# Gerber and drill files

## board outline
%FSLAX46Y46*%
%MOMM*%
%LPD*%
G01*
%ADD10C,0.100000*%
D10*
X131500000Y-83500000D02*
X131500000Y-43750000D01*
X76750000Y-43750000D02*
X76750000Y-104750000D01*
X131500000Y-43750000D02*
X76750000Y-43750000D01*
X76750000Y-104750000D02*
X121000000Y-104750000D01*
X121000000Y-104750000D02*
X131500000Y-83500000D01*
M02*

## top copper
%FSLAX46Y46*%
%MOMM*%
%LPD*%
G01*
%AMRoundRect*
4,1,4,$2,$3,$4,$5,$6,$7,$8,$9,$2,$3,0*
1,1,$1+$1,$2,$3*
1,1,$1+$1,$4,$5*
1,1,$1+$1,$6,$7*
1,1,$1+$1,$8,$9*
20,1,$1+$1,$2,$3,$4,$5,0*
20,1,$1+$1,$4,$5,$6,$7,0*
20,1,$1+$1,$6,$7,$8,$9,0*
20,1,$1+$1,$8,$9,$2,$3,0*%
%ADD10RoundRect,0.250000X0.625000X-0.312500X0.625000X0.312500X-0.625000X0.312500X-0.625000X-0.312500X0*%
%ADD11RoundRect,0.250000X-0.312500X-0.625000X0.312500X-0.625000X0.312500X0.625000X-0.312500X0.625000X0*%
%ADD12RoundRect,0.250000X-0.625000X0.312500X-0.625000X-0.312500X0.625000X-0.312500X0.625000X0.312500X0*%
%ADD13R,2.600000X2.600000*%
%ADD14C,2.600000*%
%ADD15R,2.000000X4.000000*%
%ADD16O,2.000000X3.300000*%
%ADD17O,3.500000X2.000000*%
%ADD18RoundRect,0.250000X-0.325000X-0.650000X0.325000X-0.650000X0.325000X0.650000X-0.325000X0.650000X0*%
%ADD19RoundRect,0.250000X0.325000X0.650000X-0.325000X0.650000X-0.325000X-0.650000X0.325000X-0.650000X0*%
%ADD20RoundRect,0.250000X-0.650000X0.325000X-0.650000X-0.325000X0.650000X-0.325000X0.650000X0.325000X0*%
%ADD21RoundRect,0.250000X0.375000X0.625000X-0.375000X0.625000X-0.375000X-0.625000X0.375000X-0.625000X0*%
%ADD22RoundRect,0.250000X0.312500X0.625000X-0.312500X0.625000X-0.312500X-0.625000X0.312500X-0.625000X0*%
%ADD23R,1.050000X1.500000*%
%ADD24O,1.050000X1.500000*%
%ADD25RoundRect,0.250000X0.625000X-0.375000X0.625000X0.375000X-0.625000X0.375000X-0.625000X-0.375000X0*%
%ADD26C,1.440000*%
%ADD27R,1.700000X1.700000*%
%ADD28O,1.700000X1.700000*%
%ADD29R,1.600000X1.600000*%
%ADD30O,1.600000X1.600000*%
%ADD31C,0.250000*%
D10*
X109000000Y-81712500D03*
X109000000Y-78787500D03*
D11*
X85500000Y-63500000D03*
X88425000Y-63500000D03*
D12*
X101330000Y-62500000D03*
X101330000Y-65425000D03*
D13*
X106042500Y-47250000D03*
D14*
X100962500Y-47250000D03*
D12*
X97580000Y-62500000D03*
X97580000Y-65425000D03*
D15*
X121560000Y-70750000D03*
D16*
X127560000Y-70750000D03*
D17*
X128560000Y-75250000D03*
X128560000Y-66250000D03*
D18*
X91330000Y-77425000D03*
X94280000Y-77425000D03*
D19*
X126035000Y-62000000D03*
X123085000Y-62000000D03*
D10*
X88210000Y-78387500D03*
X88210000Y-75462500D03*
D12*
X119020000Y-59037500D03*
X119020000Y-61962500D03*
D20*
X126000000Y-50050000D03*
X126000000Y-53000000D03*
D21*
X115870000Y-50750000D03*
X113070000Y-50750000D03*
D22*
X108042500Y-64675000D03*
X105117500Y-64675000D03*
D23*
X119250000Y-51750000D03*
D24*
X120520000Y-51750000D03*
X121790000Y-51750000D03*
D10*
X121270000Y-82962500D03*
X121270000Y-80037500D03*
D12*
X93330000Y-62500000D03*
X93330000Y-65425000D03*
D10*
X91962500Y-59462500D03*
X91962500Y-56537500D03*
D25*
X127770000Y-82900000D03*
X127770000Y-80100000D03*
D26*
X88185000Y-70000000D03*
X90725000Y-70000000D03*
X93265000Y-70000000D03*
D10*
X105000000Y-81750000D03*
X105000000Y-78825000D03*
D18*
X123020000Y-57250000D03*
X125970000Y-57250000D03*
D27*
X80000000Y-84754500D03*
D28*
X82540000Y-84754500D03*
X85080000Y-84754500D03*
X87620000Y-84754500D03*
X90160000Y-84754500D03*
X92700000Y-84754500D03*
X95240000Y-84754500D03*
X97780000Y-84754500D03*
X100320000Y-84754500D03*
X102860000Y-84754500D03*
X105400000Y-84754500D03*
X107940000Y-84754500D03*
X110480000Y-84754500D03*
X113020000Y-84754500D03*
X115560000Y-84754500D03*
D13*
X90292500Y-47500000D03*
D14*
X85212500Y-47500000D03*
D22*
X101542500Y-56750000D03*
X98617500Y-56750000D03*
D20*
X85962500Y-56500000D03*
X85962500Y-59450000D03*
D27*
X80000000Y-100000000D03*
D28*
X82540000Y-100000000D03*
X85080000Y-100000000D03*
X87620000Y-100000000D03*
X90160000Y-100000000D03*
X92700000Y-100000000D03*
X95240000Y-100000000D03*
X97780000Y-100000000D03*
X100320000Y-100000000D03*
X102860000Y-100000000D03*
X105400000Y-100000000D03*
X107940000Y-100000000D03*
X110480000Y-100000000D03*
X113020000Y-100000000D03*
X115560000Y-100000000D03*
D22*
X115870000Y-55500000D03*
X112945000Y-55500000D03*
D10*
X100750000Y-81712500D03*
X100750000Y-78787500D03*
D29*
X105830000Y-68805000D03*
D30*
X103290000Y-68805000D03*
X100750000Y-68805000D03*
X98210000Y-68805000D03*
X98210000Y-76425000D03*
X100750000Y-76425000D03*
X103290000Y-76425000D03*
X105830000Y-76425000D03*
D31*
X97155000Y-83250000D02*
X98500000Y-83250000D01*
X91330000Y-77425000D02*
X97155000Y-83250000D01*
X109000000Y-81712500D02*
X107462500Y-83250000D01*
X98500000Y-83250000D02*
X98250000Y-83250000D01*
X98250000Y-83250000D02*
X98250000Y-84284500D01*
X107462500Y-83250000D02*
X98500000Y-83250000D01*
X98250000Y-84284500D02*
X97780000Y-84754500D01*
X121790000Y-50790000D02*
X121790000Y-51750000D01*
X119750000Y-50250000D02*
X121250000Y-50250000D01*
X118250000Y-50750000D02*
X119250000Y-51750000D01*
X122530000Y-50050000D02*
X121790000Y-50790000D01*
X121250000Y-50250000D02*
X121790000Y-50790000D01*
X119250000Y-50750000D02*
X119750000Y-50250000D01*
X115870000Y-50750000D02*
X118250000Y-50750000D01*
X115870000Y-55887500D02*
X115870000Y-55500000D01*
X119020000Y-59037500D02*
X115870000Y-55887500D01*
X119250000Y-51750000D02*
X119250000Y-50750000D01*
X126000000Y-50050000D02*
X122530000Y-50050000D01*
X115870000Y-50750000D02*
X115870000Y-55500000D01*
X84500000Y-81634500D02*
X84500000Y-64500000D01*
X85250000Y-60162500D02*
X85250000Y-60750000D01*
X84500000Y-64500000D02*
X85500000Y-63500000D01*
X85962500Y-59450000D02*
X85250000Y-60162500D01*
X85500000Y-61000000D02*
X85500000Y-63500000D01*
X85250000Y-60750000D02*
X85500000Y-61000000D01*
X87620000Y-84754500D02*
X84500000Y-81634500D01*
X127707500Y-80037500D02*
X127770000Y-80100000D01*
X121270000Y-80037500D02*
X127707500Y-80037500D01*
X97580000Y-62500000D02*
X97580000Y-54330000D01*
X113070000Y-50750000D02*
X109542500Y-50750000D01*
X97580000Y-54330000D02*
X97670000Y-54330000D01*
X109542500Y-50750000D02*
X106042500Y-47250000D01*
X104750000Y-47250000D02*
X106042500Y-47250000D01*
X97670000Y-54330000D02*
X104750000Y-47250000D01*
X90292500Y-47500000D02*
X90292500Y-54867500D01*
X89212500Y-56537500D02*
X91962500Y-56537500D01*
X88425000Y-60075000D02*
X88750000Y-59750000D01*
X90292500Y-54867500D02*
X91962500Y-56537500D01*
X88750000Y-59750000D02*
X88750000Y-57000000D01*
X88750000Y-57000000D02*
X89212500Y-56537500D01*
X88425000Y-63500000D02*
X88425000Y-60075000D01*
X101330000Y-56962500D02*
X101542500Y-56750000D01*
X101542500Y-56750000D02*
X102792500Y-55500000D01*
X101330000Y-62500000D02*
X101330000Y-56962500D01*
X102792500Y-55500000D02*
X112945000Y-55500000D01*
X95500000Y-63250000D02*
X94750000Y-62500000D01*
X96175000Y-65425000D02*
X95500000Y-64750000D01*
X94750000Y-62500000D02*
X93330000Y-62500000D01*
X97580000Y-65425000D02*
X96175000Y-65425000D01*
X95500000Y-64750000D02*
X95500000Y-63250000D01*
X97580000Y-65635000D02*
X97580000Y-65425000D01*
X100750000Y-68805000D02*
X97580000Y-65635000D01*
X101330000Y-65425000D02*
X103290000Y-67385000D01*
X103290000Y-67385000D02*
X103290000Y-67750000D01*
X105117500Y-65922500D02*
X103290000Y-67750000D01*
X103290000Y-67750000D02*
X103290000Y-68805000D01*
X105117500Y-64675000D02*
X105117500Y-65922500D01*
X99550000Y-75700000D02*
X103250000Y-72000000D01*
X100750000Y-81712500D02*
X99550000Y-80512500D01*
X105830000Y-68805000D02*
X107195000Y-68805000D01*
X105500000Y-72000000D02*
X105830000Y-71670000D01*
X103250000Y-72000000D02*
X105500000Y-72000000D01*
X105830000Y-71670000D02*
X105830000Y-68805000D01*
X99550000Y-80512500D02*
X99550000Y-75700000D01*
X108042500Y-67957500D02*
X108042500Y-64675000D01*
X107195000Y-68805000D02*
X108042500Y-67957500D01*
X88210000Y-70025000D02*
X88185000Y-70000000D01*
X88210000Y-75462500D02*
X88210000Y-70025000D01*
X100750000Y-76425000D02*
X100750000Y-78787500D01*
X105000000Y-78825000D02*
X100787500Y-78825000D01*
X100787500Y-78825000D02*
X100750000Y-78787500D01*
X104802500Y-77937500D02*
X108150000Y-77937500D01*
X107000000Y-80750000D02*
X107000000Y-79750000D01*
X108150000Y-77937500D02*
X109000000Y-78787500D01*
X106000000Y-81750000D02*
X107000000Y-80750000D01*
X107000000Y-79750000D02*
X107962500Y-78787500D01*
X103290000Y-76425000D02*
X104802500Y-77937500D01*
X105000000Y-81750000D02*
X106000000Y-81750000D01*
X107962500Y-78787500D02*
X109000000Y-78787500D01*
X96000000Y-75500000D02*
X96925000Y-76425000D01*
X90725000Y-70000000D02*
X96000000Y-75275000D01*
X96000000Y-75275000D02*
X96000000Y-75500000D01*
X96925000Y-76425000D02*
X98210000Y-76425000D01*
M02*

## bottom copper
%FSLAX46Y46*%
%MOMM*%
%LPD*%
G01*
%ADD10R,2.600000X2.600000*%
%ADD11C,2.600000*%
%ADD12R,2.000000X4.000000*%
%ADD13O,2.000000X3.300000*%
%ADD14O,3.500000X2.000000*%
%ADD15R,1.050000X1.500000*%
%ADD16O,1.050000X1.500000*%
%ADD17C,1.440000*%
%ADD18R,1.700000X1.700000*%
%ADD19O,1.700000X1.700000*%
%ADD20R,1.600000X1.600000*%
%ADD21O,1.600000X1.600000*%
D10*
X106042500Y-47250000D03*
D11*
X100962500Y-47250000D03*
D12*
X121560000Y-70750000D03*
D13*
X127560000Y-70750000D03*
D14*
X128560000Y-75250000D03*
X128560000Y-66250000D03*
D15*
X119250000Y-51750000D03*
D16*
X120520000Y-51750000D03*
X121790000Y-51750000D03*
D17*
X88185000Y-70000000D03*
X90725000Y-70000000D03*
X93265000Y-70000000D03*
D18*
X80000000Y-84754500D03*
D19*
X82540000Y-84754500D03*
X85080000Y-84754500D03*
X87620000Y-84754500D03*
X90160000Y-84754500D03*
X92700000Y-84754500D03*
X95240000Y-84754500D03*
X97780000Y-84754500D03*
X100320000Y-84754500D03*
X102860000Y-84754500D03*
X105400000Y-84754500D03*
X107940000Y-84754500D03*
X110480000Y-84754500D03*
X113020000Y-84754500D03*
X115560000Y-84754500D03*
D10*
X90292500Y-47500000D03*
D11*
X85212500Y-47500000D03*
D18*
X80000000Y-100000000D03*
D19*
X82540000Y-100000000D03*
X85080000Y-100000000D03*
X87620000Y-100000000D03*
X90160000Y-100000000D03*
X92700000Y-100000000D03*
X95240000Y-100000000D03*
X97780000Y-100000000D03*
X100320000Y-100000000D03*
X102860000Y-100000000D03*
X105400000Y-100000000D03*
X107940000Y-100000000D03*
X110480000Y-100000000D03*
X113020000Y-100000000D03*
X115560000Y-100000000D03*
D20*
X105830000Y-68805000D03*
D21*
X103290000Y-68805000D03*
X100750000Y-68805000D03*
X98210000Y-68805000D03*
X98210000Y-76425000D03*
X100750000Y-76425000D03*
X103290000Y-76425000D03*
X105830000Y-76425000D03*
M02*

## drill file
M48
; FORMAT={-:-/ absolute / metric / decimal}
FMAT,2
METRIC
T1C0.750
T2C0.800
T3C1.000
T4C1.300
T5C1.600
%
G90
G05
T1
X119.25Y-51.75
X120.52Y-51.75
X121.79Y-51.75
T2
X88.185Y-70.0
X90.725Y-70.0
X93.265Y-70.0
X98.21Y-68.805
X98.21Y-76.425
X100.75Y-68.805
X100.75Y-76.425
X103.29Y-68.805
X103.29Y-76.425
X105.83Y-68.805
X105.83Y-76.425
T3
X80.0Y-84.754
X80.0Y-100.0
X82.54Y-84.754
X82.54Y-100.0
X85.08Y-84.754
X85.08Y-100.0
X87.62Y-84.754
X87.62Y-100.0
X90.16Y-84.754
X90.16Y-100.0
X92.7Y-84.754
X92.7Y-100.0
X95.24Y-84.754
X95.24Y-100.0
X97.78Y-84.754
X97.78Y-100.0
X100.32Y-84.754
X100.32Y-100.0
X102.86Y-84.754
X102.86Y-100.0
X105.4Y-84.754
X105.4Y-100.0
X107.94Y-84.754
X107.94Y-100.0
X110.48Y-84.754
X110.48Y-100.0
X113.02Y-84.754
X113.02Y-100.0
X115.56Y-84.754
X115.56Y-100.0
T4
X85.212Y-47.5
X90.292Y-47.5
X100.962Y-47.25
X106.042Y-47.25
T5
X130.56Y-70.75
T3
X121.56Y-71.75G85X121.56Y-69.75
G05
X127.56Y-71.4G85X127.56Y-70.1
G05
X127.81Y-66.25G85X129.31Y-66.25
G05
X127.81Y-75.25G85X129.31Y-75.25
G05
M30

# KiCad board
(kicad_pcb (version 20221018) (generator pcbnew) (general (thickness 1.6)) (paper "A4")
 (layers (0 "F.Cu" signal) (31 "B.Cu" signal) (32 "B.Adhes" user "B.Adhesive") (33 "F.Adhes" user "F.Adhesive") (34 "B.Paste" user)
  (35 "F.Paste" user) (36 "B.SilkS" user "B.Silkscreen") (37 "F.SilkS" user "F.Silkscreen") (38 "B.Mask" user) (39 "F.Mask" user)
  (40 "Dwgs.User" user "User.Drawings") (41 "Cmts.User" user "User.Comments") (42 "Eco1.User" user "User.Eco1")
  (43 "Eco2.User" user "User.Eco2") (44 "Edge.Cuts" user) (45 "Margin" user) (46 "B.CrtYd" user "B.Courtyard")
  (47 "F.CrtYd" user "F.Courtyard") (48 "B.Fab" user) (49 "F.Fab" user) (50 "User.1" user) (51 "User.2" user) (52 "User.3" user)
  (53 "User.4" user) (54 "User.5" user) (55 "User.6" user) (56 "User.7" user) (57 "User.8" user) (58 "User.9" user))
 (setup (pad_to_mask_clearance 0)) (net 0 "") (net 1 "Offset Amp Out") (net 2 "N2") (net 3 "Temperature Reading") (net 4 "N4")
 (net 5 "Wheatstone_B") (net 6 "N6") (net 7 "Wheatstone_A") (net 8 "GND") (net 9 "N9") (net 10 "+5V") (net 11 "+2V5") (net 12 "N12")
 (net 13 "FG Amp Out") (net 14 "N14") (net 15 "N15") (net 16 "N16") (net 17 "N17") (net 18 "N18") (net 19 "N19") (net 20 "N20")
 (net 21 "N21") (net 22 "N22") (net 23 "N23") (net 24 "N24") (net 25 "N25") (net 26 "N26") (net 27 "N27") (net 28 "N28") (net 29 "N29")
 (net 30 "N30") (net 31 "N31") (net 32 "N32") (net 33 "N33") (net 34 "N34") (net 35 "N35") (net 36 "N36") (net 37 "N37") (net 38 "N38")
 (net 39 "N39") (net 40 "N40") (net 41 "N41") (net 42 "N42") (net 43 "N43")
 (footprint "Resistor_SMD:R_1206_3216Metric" (layer "F.Cu") (at 109 80.25 90)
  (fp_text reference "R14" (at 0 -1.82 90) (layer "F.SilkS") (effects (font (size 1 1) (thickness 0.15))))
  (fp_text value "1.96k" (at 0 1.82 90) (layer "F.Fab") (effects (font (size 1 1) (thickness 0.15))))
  (pad "1" smd roundrect (at -1.4625 0 90) (size 1.125 1.75) (layers "F.Cu" "F.Paste" "F.Mask") (roundrect_rratio 0.222222)
   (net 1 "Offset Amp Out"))
  (pad "2" smd roundrect (at 1.4625 0 90) (size 1.125 1.75) (layers "F.Cu" "F.Paste" "F.Mask") (roundrect_rratio 0.222222) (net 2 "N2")))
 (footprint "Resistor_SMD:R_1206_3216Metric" (layer "F.Cu") (at 86.9625 63.5)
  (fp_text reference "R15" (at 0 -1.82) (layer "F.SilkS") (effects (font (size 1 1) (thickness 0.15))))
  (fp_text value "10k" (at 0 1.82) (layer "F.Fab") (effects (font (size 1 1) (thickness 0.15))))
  (pad "1" smd roundrect (at -1.4625 0) (size 1.125 1.75) (layers "F.Cu" "F.Paste" "F.Mask") (roundrect_rratio 0.222222)
   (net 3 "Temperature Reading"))
  (pad "2" smd roundrect (at 1.4625 0) (size 1.125 1.75) (layers "F.Cu" "F.Paste" "F.Mask") (roundrect_rratio 0.222222) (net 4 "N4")))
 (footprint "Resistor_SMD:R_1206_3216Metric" (layer "F.Cu") (at 101.33 63.9625 -90)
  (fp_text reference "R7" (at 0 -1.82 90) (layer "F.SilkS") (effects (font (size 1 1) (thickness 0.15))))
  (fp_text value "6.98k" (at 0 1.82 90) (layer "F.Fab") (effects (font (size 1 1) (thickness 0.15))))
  (pad "1" smd roundrect (at -1.4625 0 270) (size 1.125 1.75) (layers "F.Cu" "F.Paste" "F.Mask") (roundrect_rratio 0.222222)
   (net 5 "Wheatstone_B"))
  (pad "2" smd roundrect (at 1.4625 0 270) (size 1.125 1.75) (layers "F.Cu" "F.Paste" "F.Mask") (roundrect_rratio 0.222222) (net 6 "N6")))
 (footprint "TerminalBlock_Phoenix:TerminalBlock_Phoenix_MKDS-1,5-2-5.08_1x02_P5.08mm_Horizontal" (layer "F.Cu") (at 106.0425 47.25 180)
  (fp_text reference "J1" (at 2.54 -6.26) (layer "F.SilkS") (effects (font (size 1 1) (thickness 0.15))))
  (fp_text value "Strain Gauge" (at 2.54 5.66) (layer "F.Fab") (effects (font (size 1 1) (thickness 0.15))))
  (pad "1" thru_hole rect (at 0 0 180) (size 2.6 2.6) (drill 1.3) (layers "*.Cu" "*.Mask") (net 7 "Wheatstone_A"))
  (pad "2" thru_hole circle (at 5.08 0 180) (size 2.6 2.6) (drill 1.3) (layers "*.Cu" "*.Mask") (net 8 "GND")))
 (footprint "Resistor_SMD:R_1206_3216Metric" (layer "F.Cu") (at 97.58 63.9625 -90)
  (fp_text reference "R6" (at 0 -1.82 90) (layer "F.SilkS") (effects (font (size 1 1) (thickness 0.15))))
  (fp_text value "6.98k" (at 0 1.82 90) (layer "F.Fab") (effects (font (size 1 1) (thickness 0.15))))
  (pad "1" smd roundrect (at -1.4625 0 270) (size 1.125 1.75) (layers "F.Cu" "F.Paste" "F.Mask") (roundrect_rratio 0.222222)
   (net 7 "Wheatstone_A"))
  (pad "2" smd roundrect (at 1.4625 0 270) (size 1.125 1.75) (layers "F.Cu" "F.Paste" "F.Mask") (roundrect_rratio 0.222222) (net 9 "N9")))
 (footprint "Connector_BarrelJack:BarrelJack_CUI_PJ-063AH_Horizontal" (layer "F.Cu") (at 121.56 70.75 90)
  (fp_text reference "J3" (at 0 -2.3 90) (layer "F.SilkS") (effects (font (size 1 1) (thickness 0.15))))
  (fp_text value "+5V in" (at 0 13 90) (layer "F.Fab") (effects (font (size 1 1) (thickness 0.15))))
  (pad "" np_thru_hole circle (at 0 9 90) (size 1.6 1.6) (drill 1.6) (layers "*.Cu" "*.Mask"))
  (pad "1" thru_hole rect (at 0 0 90) (size 4 2) (drill oval 3 1) (layers "*.Cu" "*.Mask") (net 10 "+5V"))
  (pad "2" thru_hole oval (at 0 6 90) (size 3.3 2) (drill oval 2.3 1) (layers "*.Cu" "*.Mask") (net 8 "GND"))
  (pad "MP" thru_hole oval (at -4.5 7 90) (size 2 3.5) (drill oval 1 2.5) (layers "*.Cu" "*.Mask"))
  (pad "MP" thru_hole oval (at 4.5 7 90) (size 2 3.5) (drill oval 1 2.5) (layers "*.Cu" "*.Mask")))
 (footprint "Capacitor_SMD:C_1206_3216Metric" (layer "F.Cu") (at 92.805 77.425)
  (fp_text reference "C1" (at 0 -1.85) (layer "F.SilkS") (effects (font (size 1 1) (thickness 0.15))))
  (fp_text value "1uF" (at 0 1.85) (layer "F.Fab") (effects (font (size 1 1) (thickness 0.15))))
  (pad "1" smd roundrect (at -1.475 0) (size 1.15 1.8) (layers "F.Cu" "F.Paste" "F.Mask") (roundrect_rratio 0.217391)
   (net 1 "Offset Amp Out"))
  (pad "2" smd roundrect (at 1.475 0) (size 1.15 1.8) (layers "F.Cu" "F.Paste" "F.Mask") (roundrect_rratio 0.217391) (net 8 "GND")))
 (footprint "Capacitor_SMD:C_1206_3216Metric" (layer "F.Cu") (at 124.56 62 180)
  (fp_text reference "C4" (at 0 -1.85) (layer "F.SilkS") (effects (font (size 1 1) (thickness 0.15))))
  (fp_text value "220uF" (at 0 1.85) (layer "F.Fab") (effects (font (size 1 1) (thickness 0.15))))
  (pad "1" smd roundrect (at -1.475 0 180) (size 1.15 1.8) (layers "F.Cu" "F.Paste" "F.Mask") (roundrect_rratio 0.217391) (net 8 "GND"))
  (pad "2" smd roundrect (at 1.475 0 180) (size 1.15 1.8) (layers "F.Cu" "F.Paste" "F.Mask") (roundrect_rratio 0.217391) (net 10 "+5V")))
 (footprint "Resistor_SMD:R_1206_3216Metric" (layer "F.Cu") (at 88.21 76.925 90)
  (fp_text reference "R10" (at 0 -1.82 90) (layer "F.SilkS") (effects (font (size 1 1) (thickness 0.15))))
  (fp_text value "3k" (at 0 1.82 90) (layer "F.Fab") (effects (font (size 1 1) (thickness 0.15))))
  (pad "1" smd roundrect (at -1.4625 0 90) (size 1.125 1.75) (layers "F.Cu" "F.Paste" "F.Mask") (roundrect_rratio 0.222222) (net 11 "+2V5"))
  (pad "2" smd roundrect (at 1.4625 0 90) (size 1.125 1.75) (layers "F.Cu" "F.Paste" "F.Mask") (roundrect_rratio 0.222222) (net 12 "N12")))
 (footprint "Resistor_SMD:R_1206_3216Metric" (layer "F.Cu") (at 119.02 60.5 -90)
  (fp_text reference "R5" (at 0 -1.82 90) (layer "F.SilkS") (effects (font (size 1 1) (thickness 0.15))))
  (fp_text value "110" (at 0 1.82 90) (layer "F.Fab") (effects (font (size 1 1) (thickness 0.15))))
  (pad "1" smd roundrect (at -1.4625 0 270) (size 1.125 1.75) (layers "F.Cu" "F.Paste" "F.Mask") (roundrect_rratio 0.222222) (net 11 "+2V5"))
  (pad "2" smd roundrect (at 1.4625 0 270) (size 1.125 1.75) (layers "F.Cu" "F.Paste" "F.Mask") (roundrect_rratio 0.222222) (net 10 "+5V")))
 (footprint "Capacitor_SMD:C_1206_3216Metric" (layer "F.Cu") (at 126 51.525 -90)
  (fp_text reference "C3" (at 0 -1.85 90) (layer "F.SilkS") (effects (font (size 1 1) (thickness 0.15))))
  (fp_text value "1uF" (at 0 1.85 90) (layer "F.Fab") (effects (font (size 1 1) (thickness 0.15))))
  (pad "1" smd roundrect (at -1.475 0 270) (size 1.15 1.8) (layers "F.Cu" "F.Paste" "F.Mask") (roundrect_rratio 0.217391) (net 11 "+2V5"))
  (pad "2" smd roundrect (at 1.475 0 270) (size 1.15 1.8) (layers "F.Cu" "F.Paste" "F.Mask") (roundrect_rratio 0.217391) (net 8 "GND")))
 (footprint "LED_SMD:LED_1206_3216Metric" (layer "F.Cu") (at 114.47 50.75 180)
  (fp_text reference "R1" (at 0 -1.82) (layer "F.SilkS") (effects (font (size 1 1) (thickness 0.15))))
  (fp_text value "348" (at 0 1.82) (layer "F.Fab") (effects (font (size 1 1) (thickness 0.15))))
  (pad "1" smd roundrect (at -1.4 0 180) (size 1.25 1.75) (layers "F.Cu" "F.Paste" "F.Mask") (roundrect_rratio 0.2) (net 11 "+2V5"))
  (pad "2" smd roundrect (at 1.4 0 180) (size 1.25 1.75) (layers "F.Cu" "F.Paste" "F.Mask") (roundrect_rratio 0.2) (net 7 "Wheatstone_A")))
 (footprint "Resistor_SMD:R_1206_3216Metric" (layer "F.Cu") (at 106.58 64.675 180)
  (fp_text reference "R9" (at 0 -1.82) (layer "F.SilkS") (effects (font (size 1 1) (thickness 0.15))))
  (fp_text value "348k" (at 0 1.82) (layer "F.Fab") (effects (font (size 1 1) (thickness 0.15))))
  (pad "1" smd roundrect (at -1.4625 0 180) (size 1.125 1.75) (layers "F.Cu" "F.Paste" "F.Mask") (roundrect_rratio 0.222222)
   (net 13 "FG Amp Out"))
  (pad "2" smd roundrect (at 1.4625 0 180) (size 1.125 1.75) (layers "F.Cu" "F.Paste" "F.Mask") (roundrect_rratio 0.222222) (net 6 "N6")))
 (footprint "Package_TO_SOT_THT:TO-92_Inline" (layer "F.Cu") (at 119.25 51.75)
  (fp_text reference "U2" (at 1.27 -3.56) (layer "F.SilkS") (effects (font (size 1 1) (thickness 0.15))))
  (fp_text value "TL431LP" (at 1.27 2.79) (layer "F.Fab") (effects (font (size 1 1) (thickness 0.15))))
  (pad "1" thru_hole rect (at 0 0) (size 1.05 1.5) (drill 0.75) (layers "*.Cu" "*.Mask") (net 11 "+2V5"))
  (pad "2" thru_hole oval (at 1.27 0) (size 1.05 1.5) (drill 0.75) (layers "*.Cu" "*.Mask") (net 8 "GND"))
  (pad "3" thru_hole oval (at 2.54 0) (size 1.05 1.5) (drill 0.75) (layers "*.Cu" "*.Mask") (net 11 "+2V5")))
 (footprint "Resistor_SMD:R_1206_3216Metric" (layer "F.Cu") (at 121.27 81.5 90)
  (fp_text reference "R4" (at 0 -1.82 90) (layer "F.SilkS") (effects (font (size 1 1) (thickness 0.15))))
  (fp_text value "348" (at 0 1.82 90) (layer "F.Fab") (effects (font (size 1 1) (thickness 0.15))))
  (pad "1" smd roundrect (at -1.4625 0 90) (size 1.125 1.75) (layers "F.Cu" "F.Paste" "F.Mask") (roundrect_rratio 0.222222) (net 10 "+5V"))
  (pad "2" smd roundrect (at 1.4625 0 90) (size 1.125 1.75) (layers "F.Cu" "F.Paste" "F.Mask") (roundrect_rratio 0.222222) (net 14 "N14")))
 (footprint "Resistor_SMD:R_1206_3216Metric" (layer "F.Cu") (at 93.33 63.9625 -90)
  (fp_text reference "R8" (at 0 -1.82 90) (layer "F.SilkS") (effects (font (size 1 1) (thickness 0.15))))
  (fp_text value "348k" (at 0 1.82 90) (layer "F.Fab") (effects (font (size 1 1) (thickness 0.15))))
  (pad "1" smd roundrect (at -1.4625 0 270) (size 1.125 1.75) (layers "F.Cu" "F.Paste" "F.Mask") (roundrect_rratio 0.222222) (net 9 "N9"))
  (pad "2" smd roundrect (at 1.4625 0 270) (size 1.125 1.75) (layers "F.Cu" "F.Paste" "F.Mask") (roundrect_rratio 0.222222) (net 8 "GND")))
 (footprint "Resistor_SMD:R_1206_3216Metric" (layer "F.Cu") (at 91.9625 58 90)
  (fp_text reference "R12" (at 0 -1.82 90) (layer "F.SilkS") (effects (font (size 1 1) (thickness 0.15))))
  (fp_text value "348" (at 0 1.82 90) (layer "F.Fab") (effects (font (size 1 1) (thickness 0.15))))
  (pad "1" smd roundrect (at -1.4625 0 90) (size 1.125 1.75) (layers "F.Cu" "F.Paste" "F.Mask") (roundrect_rratio 0.222222) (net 10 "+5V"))
  (pad "2" smd roundrect (at 1.4625 0 90) (size 1.125 1.75) (layers "F.Cu" "F.Paste" "F.Mask") (roundrect_rratio 0.222222) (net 4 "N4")))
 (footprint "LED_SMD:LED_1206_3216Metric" (layer "F.Cu") (at 127.77 81.5 90)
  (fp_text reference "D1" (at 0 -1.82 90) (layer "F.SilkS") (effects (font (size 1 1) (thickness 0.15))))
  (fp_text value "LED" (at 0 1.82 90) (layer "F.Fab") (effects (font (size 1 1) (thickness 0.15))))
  (pad "1" smd roundrect (at -1.4 0 90) (size 1.25 1.75) (layers "F.Cu" "F.Paste" "F.Mask") (roundrect_rratio 0.2) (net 8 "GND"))
  (pad "2" smd roundrect (at 1.4 0 90) (size 1.25 1.75) (layers "F.Cu" "F.Paste" "F.Mask") (roundrect_rratio 0.2) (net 14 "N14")))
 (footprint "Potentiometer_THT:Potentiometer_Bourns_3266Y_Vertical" (layer "F.Cu") (at 88.185 70 180)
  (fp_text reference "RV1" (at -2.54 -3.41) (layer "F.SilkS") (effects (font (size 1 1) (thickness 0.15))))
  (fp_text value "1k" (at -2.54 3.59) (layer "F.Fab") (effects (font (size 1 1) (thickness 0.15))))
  (pad "1" thru_hole circle (at 0 0 180) (size 1.44 1.44) (drill 0.8) (layers "*.Cu" "*.Mask") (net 12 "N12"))
  (pad "2" thru_hole circle (at -2.54 0 180) (size 1.44 1.44) (drill 0.8) (layers "*.Cu" "*.Mask") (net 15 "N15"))
  (pad "3" thru_hole circle (at -5.08 0 180) (size 1.44 1.44) (drill 0.8) (layers "*.Cu" "*.Mask") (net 8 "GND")))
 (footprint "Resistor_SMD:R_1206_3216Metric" (layer "F.Cu") (at 105 80.2875 90)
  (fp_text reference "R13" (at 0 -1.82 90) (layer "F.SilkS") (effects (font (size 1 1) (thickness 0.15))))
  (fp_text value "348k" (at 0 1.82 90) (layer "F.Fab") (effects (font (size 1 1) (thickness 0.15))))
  (pad "1" smd roundrect (at -1.4625 0 90) (size 1.125 1.75) (layers "F.Cu" "F.Paste" "F.Mask") (roundrect_rratio 0.222222) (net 2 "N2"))
  (pad "2" smd roundrect (at 1.4625 0 90) (size 1.125 1.75) (layers "F.Cu" "F.Paste" "F.Mask") (roundrect_rratio 0.222222) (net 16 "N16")))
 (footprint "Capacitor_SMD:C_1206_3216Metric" (layer "F.Cu") (at 124.495 57.25)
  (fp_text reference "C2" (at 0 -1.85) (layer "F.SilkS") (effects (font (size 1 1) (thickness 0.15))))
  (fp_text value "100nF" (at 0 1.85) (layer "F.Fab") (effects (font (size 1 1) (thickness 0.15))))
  (pad "1" smd roundrect (at -1.475 0) (size 1.15 1.8) (layers "F.Cu" "F.Paste" "F.Mask") (roundrect_rratio 0.217391) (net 10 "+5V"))
  (pad "2" smd roundrect (at 1.475 0) (size 1.15 1.8) (layers "F.Cu" "F.Paste" "F.Mask") (roundrect_rratio 0.217391) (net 8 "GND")))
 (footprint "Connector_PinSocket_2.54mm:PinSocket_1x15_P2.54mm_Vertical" (layer "F.Cu") (at 80 84.7545 90)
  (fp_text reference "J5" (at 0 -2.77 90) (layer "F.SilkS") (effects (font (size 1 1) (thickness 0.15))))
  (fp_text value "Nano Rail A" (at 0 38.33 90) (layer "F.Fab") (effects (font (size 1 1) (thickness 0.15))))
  (pad "1" thru_hole rect (at 0 0 90) (size 1.7 1.7) (drill 1) (layers "*.Cu" "*.Mask") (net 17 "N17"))
  (pad "2" thru_hole oval (at 0 2.54 90) (size 1.7 1.7) (drill 1) (layers "*.Cu" "*.Mask") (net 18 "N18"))
  (pad "3" thru_hole oval (at 0 5.08 90) (size 1.7 1.7) (drill 1) (layers "*.Cu" "*.Mask") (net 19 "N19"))
  (pad "4" thru_hole oval (at 0 7.62 90) (size 1.7 1.7) (drill 1) (layers "*.Cu" "*.Mask") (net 3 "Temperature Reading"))
  (pad "5" thru_hole oval (at 0 10.16 90) (size 1.7 1.7) (drill 1) (layers "*.Cu" "*.Mask") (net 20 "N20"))
  (pad "6" thru_hole oval (at 0 12.7 90) (size 1.7 1.7) (drill 1) (layers "*.Cu" "*.Mask") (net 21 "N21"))
  (pad "7" thru_hole oval (at 0 15.24 90) (size 1.7 1.7) (drill 1) (layers "*.Cu" "*.Mask") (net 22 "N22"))
  (pad "8" thru_hole oval (at 0 17.78 90) (size 1.7 1.7) (drill 1) (layers "*.Cu" "*.Mask") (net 1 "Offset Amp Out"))
  (pad "9" thru_hole oval (at 0 20.32 90) (size 1.7 1.7) (drill 1) (layers "*.Cu" "*.Mask") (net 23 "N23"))
  (pad "10" thru_hole oval (at 0 22.86 90) (size 1.7 1.7) (drill 1) (layers "*.Cu" "*.Mask") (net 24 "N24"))
  (pad "11" thru_hole oval (at 0 25.4 90) (size 1.7 1.7) (drill 1) (layers "*.Cu" "*.Mask") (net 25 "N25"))
  (pad "12" thru_hole oval (at 0 27.94 90) (size 1.7 1.7) (drill 1) (layers "*.Cu" "*.Mask") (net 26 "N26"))
  (pad "13" thru_hole oval (at 0 30.48 90) (size 1.7 1.7) (drill 1) (layers "*.Cu" "*.Mask") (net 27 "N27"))
  (pad "14" thru_hole oval (at 0 33.02 90) (size 1.7 1.7) (drill 1) (layers "*.Cu" "*.Mask") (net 8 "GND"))
  (pad "15" thru_hole oval (at 0 35.56 90) (size 1.7 1.7) (drill 1) (layers "*.Cu" "*.Mask") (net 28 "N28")))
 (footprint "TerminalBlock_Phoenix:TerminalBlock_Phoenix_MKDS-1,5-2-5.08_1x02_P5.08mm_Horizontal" (layer "F.Cu") (at 90.2925 47.5 180)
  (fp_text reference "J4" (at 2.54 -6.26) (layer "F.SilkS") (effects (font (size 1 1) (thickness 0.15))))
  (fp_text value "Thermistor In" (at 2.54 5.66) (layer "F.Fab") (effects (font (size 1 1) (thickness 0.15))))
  (pad "1" thru_hole rect (at 0 0 180) (size 2.6 2.6) (drill 1.3) (layers "*.Cu" "*.Mask") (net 4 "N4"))
  (pad "2" thru_hole circle (at 5.08 0 180) (size 2.6 2.6) (drill 1.3) (layers "*.Cu" "*.Mask") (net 8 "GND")))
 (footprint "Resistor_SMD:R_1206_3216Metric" (layer "F.Cu") (at 100.08 56.75 180)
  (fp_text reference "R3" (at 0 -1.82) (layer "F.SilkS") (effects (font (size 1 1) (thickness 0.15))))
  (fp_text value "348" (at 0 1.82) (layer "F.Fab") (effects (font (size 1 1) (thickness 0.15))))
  (pad "1" smd roundrect (at -1.4625 0 180) (size 1.125 1.75) (layers "F.Cu" "F.Paste" "F.Mask") (roundrect_rratio 0.222222)
   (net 5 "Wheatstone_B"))
  (pad "2" smd roundrect (at 1.4625 0 180) (size 1.125 1.75) (layers "F.Cu" "F.Paste" "F.Mask") (roundrect_rratio 0.222222) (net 8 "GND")))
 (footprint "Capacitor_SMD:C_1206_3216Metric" (layer "F.Cu") (at 85.9625 57.975 -90)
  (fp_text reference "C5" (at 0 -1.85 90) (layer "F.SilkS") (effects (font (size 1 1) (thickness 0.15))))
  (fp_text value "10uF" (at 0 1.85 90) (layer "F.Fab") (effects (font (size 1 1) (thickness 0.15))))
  (pad "1" smd roundrect (at -1.475 0 270) (size 1.15 1.8) (layers "F.Cu" "F.Paste" "F.Mask") (roundrect_rratio 0.217391) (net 8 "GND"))
  (pad "2" smd roundrect (at 1.475 0 270) (size 1.15 1.8) (layers "F.Cu" "F.Paste" "F.Mask") (roundrect_rratio 0.217391)
   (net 3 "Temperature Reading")))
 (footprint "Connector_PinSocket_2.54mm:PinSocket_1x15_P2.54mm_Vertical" (layer "F.Cu") (at 80 100 90)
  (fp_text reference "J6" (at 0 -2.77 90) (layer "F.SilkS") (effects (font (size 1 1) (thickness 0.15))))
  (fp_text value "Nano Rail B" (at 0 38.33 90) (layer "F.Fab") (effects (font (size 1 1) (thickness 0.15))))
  (pad "1" thru_hole rect (at 0 0 90) (size 1.7 1.7) (drill 1) (layers "*.Cu" "*.Mask") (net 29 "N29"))
  (pad "2" thru_hole oval (at 0 2.54 90) (size 1.7 1.7) (drill 1) (layers "*.Cu" "*.Mask") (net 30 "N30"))
  (pad "3" thru_hole oval (at 0 5.08 90) (size 1.7 1.7) (drill 1) (layers "*.Cu" "*.Mask") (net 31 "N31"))
  (pad "4" thru_hole oval (at 0 7.62 90) (size 1.7 1.7) (drill 1) (layers "*.Cu" "*.Mask") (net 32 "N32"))
  (pad "5" thru_hole oval (at 0 10.16 90) (size 1.7 1.7) (drill 1) (layers "*.Cu" "*.Mask") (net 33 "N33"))
  (pad "6" thru_hole oval (at 0 12.7 90) (size 1.7 1.7) (drill 1) (layers "*.Cu" "*.Mask") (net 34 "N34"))
  (pad "7" thru_hole oval (at 0 15.24 90) (size 1.7 1.7) (drill 1) (layers "*.Cu" "*.Mask") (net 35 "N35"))
  (pad "8" thru_hole oval (at 0 17.78 90) (size 1.7 1.7) (drill 1) (layers "*.Cu" "*.Mask") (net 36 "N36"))
  (pad "9" thru_hole oval (at 0 20.32 90) (size 1.7 1.7) (drill 1) (layers "*.Cu" "*.Mask") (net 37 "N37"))
  (pad "10" thru_hole oval (at 0 22.86 90) (size 1.7 1.7) (drill 1) (layers "*.Cu" "*.Mask") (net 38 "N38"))
  (pad "11" thru_hole oval (at 0 25.4 90) (size 1.7 1.7) (drill 1) (layers "*.Cu" "*.Mask") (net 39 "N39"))
  (pad "12" thru_hole oval (at 0 27.94 90) (size 1.7 1.7) (drill 1) (layers "*.Cu" "*.Mask") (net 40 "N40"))
  (pad "13" thru_hole oval (at 0 30.48 90) (size 1.7 1.7) (drill 1) (layers "*.Cu" "*.Mask") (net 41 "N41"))
  (pad "14" thru_hole oval (at 0 33.02 90) (size 1.7 1.7) (drill 1) (layers "*.Cu" "*.Mask") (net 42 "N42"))
  (pad "15" thru_hole oval (at 0 35.56 90) (size 1.7 1.7) (drill 1) (layers "*.Cu" "*.Mask") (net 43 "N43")))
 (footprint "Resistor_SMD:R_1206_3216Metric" (layer "F.Cu") (at 114.4075 55.5 180)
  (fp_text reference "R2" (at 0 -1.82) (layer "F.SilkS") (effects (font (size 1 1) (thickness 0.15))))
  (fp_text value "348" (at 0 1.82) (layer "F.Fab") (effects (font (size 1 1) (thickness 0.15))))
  (pad "1" smd roundrect (at -1.4625 0 180) (size 1.125 1.75) (layers "F.Cu" "F.Paste" "F.Mask") (roundrect_rratio 0.222222) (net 11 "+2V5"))
  (pad "2" smd roundrect (at 1.4625 0 180) (size 1.125 1.75) (layers "F.Cu" "F.Paste" "F.Mask") (roundrect_rratio 0.222222)
   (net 5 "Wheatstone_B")))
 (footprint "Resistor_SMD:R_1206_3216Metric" (layer "F.Cu") (at 100.75 80.25 90)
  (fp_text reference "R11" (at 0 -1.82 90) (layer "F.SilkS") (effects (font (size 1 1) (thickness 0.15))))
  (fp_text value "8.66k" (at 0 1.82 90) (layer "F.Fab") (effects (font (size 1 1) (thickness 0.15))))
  (pad "1" smd roundrect (at -1.4625 0 90) (size 1.125 1.75) (layers "F.Cu" "F.Paste" "F.Mask") (roundrect_rratio 0.222222)
   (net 13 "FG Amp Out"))
  (pad "2" smd roundrect (at 1.4625 0 90) (size 1.125 1.75) (layers "F.Cu" "F.Paste" "F.Mask") (roundrect_rratio 0.222222) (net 16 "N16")))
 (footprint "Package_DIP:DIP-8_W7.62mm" (layer "F.Cu") (at 105.83 68.805 -90)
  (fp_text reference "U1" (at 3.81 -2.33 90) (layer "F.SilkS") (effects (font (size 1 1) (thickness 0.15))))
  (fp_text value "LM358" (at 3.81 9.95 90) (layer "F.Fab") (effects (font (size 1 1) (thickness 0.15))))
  (pad "1" thru_hole rect (at 0 0 270) (size 1.6 1.6) (drill 0.8) (layers "*.Cu" "*.Mask") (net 13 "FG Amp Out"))
  (pad "2" thru_hole oval (at 0 2.54 270) (size 1.6 1.6) (drill 0.8) (layers "*.Cu" "*.Mask") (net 6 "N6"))
  (pad "3" thru_hole oval (at 0 5.08 270) (size 1.6 1.6) (drill 0.8) (layers "*.Cu" "*.Mask") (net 9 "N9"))
  (pad "4" thru_hole oval (at 0 7.62 270) (size 1.6 1.6) (drill 0.8) (layers "*.Cu" "*.Mask") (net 8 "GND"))
  (pad "5" thru_hole oval (at 7.62 7.62 270) (size 1.6 1.6) (drill 0.8) (layers "*.Cu" "*.Mask") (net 15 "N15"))
  (pad "6" thru_hole oval (at 7.62 5.08 270) (size 1.6 1.6) (drill 0.8) (layers "*.Cu" "*.Mask") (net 16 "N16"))
  (pad "7" thru_hole oval (at 7.62 2.54 270) (size 1.6 1.6) (drill 0.8) (layers "*.Cu" "*.Mask") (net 2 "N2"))
  (pad "8" thru_hole oval (at 7.62 0 270) (size 1.6 1.6) (drill 0.8) (layers "*.Cu" "*.Mask") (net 10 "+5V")))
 (gr_line (start 131.5 83.5) (end 131.5 43.75) (stroke (width 0.1) (type default)) (layer "Edge.Cuts"))
 (gr_line (start 76.75 43.75) (end 76.75 104.75) (stroke (width 0.1) (type default)) (layer "Edge.Cuts"))
 (gr_line (start 131.5 43.75) (end 76.75 43.75) (stroke (width 0.1) (type default)) (layer "Edge.Cuts"))
 (gr_line (start 76.75 104.75) (end 121 104.75) (stroke (width 0.1) (type default)) (layer "Edge.Cuts"))
 (gr_line (start 121 104.75) (end 131.5 83.5) (stroke (width 0.1) (type default)) (layer "Edge.Cuts"))
 (segment (start 97.155 83.25) (end 98.5 83.25) (width 0.25) (layer "F.Cu") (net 1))
 (segment (start 91.33 77.425) (end 97.155 83.25) (width 0.25) (layer "F.Cu") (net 1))
 (segment (start 109 81.7125) (end 107.4625 83.25) (width 0.25) (layer "F.Cu") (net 1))
 (segment (start 98.5 83.25) (end 98.25 83.25) (width 0.25) (layer "F.Cu") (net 1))
 (segment (start 98.25 83.25) (end 98.25 84.2845) (width 0.25) (layer "F.Cu") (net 1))
 (segment (start 107.4625 83.25) (end 98.5 83.25) (width 0.25) (layer "F.Cu") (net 1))
 (segment (start 98.25 84.2845) (end 97.78 84.7545) (width 0.25) (layer "F.Cu") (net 1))
 (segment (start 121.79 50.79) (end 121.79 51.75) (width 0.25) (layer "F.Cu") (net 11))
 (segment (start 119.75 50.25) (end 121.25 50.25) (width 0.25) (layer "F.Cu") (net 11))
 (segment (start 118.25 50.75) (end 119.25 51.75) (width 0.25) (layer "F.Cu") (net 11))
 (segment (start 122.53 50.05) (end 121.79 50.79) (width 0.25) (layer "F.Cu") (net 11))
 (segment (start 121.25 50.25) (end 121.79 50.79) (width 0.25) (layer "F.Cu") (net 11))
 (segment (start 119.25 50.75) (end 119.75 50.25) (width 0.25) (layer "F.Cu") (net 11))
 (segment (start 115.87 50.75) (end 118.25 50.75) (width 0.25) (layer "F.Cu") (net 11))
 (segment (start 115.87 55.8875) (end 115.87 55.5) (width 0.25) (layer "F.Cu") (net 11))
 (segment (start 119.02 59.0375) (end 115.87 55.8875) (width 0.25) (layer "F.Cu") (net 11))
 (segment (start 119.25 51.75) (end 119.25 50.75) (width 0.25) (layer "F.Cu") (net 11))
 (segment (start 126 50.05) (end 122.53 50.05) (width 0.25) (layer "F.Cu") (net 11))
 (segment (start 115.87 50.75) (end 115.87 55.5) (width 0.25) (layer "F.Cu") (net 11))
 (segment (start 84.5 81.6345) (end 84.5 64.5) (width 0.25) (layer "F.Cu") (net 3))
 (segment (start 85.25 60.1625) (end 85.25 60.75) (width 0.25) (layer "F.Cu") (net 3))
 (segment (start 84.5 64.5) (end 85.5 63.5) (width 0.25) (layer "F.Cu") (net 3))
 (segment (start 85.9625 59.45) (end 85.25 60.1625) (width 0.25) (layer "F.Cu") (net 3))
 (segment (start 85.5 61) (end 85.5 63.5) (width 0.25) (layer "F.Cu") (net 3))
 (segment (start 85.25 60.75) (end 85.5 61) (width 0.25) (layer "F.Cu") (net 3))
 (segment (start 87.62 84.7545) (end 84.5 81.6345) (width 0.25) (layer "F.Cu") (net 3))
 (segment (start 127.7075 80.0375) (end 127.77 80.1) (width 0.25) (layer "F.Cu") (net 14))
 (segment (start 121.27 80.0375) (end 127.7075 80.0375) (width 0.25) (layer "F.Cu") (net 14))
 (segment (start 97.58 62.5) (end 97.58 54.33) (width 0.25) (layer "F.Cu") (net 7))
 (segment (start 113.07 50.75) (end 109.5425 50.75) (width 0.25) (layer "F.Cu") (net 7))
 (segment (start 97.58 54.33) (end 97.67 54.33) (width 0.25) (layer "F.Cu") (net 7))
 (segment (start 109.5425 50.75) (end 106.0425 47.25) (width 0.25) (layer "F.Cu") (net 7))
 (segment (start 104.75 47.25) (end 106.0425 47.25) (width 0.25) (layer "F.Cu") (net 7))
 (segment (start 97.67 54.33) (end 104.75 47.25) (width 0.25) (layer "F.Cu") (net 7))
 (segment (start 90.2925 47.5) (end 90.2925 54.8675) (width 0.25) (layer "F.Cu") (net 4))
 (segment (start 89.2125 56.5375) (end 91.9625 56.5375) (width 0.25) (layer "F.Cu") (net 4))
 (segment (start 88.425 60.075) (end 88.75 59.75) (width 0.25) (layer "F.Cu") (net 4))
 (segment (start 90.2925 54.8675) (end 91.9625 56.5375) (width 0.25) (layer "F.Cu") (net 4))
 (segment (start 88.75 59.75) (end 88.75 57) (width 0.25) (layer "F.Cu") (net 4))
 (segment (start 88.75 57) (end 89.2125 56.5375) (width 0.25) (layer "F.Cu") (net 4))
 (segment (start 88.425 63.5) (end 88.425 60.075) (width 0.25) (layer "F.Cu") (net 4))
 (segment (start 101.33 56.9625) (end 101.5425 56.75) (width 0.25) (layer "F.Cu") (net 5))
 (segment (start 101.5425 56.75) (end 102.7925 55.5) (width 0.25) (layer "F.Cu") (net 5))
 (segment (start 101.33 62.5) (end 101.33 56.9625) (width 0.25) (layer "F.Cu") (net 5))
 (segment (start 102.7925 55.5) (end 112.945 55.5) (width 0.25) (layer "F.Cu") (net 5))
 (segment (start 95.5 63.25) (end 94.75 62.5) (width 0.25) (layer "F.Cu") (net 9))
 (segment (start 96.175 65.425) (end 95.5 64.75) (width 0.25) (layer "F.Cu") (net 9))
 (segment (start 94.75 62.5) (end 93.33 62.5) (width 0.25) (layer "F.Cu") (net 9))
 (segment (start 97.58 65.425) (end 96.175 65.425) (width 0.25) (layer "F.Cu") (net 9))
 (segment (start 95.5 64.75) (end 95.5 63.25) (width 0.25) (layer "F.Cu") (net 9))
 (segment (start 97.58 65.635) (end 97.58 65.425) (width 0.25) (layer "F.Cu") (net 9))
 (segment (start 100.75 68.805) (end 97.58 65.635) (width 0.25) (layer "F.Cu") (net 9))
 (segment (start 101.33 65.425) (end 103.29 67.385) (width 0.25) (layer "F.Cu") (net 6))
 (segment (start 103.29 67.385) (end 103.29 67.75) (width 0.25) (layer "F.Cu") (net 6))
 (segment (start 105.1175 65.9225) (end 103.29 67.75) (width 0.25) (layer "F.Cu") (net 6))
 (segment (start 103.29 67.75) (end 103.29 68.805) (width 0.25) (layer "F.Cu") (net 6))
 (segment (start 105.1175 64.675) (end 105.1175 65.9225) (width 0.25) (layer "F.Cu") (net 6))
 (segment (start 99.55 75.7) (end 103.25 72) (width 0.25) (layer "F.Cu") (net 13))
 (segment (start 100.75 81.7125) (end 99.55 80.5125) (width 0.25) (layer "F.Cu") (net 13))
 (segment (start 105.83 68.805) (end 107.195 68.805) (width 0.25) (layer "F.Cu") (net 13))
 (segment (start 105.5 72) (end 105.83 71.67) (width 0.25) (layer "F.Cu") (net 13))
 (segment (start 103.25 72) (end 105.5 72) (width 0.25) (layer "F.Cu") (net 13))
 (segment (start 105.83 71.67) (end 105.83 68.805) (width 0.25) (layer "F.Cu") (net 13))
 (segment (start 99.55 80.5125) (end 99.55 75.7) (width 0.25) (layer "F.Cu") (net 13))
 (segment (start 108.0425 67.9575) (end 108.0425 64.675) (width 0.25) (layer "F.Cu") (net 13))
 (segment (start 107.195 68.805) (end 108.0425 67.9575) (width 0.25) (layer "F.Cu") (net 13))
 (segment (start 88.21 70.025) (end 88.185 70) (width 0.25) (layer "F.Cu") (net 12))
 (segment (start 88.21 75.4625) (end 88.21 70.025) (width 0.25) (layer "F.Cu") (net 12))
 (segment (start 100.75 76.425) (end 100.75 78.7875) (width 0.25) (layer "F.Cu") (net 16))
 (segment (start 105 78.825) (end 100.7875 78.825) (width 0.25) (layer "F.Cu") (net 16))
 (segment (start 100.7875 78.825) (end 100.75 78.7875) (width 0.25) (layer "F.Cu") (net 16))
 (segment (start 104.8025 77.9375) (end 108.15 77.9375) (width 0.25) (layer "F.Cu") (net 2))
 (segment (start 107 80.75) (end 107 79.75) (width 0.25) (layer "F.Cu") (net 2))
 (segment (start 108.15 77.9375) (end 109 78.7875) (width 0.25) (layer "F.Cu") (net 2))
 (segment (start 106 81.75) (end 107 80.75) (width 0.25) (layer "F.Cu") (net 2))
 (segment (start 107 79.75) (end 107.9625 78.7875) (width 0.25) (layer "F.Cu") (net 2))
 (segment (start 103.29 76.425) (end 104.8025 77.9375) (width 0.25) (layer "F.Cu") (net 2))
 (segment (start 105 81.75) (end 106 81.75) (width 0.25) (layer "F.Cu") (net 2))
 (segment (start 107.9625 78.7875) (end 109 78.7875) (width 0.25) (layer "F.Cu") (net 2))
 (segment (start 96 75.5) (end 96.925 76.425) (width 0.25) (layer "F.Cu") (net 15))
 (segment (start 90.725 70) (end 96 75.275) (width 0.25) (layer "F.Cu") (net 15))
 (segment (start 96 75.275) (end 96 75.5) (width 0.25) (layer "F.Cu") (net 15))
 (segment (start 96.925 76.425) (end 98.21 76.425) (width 0.25) (layer "F.Cu") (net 15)))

